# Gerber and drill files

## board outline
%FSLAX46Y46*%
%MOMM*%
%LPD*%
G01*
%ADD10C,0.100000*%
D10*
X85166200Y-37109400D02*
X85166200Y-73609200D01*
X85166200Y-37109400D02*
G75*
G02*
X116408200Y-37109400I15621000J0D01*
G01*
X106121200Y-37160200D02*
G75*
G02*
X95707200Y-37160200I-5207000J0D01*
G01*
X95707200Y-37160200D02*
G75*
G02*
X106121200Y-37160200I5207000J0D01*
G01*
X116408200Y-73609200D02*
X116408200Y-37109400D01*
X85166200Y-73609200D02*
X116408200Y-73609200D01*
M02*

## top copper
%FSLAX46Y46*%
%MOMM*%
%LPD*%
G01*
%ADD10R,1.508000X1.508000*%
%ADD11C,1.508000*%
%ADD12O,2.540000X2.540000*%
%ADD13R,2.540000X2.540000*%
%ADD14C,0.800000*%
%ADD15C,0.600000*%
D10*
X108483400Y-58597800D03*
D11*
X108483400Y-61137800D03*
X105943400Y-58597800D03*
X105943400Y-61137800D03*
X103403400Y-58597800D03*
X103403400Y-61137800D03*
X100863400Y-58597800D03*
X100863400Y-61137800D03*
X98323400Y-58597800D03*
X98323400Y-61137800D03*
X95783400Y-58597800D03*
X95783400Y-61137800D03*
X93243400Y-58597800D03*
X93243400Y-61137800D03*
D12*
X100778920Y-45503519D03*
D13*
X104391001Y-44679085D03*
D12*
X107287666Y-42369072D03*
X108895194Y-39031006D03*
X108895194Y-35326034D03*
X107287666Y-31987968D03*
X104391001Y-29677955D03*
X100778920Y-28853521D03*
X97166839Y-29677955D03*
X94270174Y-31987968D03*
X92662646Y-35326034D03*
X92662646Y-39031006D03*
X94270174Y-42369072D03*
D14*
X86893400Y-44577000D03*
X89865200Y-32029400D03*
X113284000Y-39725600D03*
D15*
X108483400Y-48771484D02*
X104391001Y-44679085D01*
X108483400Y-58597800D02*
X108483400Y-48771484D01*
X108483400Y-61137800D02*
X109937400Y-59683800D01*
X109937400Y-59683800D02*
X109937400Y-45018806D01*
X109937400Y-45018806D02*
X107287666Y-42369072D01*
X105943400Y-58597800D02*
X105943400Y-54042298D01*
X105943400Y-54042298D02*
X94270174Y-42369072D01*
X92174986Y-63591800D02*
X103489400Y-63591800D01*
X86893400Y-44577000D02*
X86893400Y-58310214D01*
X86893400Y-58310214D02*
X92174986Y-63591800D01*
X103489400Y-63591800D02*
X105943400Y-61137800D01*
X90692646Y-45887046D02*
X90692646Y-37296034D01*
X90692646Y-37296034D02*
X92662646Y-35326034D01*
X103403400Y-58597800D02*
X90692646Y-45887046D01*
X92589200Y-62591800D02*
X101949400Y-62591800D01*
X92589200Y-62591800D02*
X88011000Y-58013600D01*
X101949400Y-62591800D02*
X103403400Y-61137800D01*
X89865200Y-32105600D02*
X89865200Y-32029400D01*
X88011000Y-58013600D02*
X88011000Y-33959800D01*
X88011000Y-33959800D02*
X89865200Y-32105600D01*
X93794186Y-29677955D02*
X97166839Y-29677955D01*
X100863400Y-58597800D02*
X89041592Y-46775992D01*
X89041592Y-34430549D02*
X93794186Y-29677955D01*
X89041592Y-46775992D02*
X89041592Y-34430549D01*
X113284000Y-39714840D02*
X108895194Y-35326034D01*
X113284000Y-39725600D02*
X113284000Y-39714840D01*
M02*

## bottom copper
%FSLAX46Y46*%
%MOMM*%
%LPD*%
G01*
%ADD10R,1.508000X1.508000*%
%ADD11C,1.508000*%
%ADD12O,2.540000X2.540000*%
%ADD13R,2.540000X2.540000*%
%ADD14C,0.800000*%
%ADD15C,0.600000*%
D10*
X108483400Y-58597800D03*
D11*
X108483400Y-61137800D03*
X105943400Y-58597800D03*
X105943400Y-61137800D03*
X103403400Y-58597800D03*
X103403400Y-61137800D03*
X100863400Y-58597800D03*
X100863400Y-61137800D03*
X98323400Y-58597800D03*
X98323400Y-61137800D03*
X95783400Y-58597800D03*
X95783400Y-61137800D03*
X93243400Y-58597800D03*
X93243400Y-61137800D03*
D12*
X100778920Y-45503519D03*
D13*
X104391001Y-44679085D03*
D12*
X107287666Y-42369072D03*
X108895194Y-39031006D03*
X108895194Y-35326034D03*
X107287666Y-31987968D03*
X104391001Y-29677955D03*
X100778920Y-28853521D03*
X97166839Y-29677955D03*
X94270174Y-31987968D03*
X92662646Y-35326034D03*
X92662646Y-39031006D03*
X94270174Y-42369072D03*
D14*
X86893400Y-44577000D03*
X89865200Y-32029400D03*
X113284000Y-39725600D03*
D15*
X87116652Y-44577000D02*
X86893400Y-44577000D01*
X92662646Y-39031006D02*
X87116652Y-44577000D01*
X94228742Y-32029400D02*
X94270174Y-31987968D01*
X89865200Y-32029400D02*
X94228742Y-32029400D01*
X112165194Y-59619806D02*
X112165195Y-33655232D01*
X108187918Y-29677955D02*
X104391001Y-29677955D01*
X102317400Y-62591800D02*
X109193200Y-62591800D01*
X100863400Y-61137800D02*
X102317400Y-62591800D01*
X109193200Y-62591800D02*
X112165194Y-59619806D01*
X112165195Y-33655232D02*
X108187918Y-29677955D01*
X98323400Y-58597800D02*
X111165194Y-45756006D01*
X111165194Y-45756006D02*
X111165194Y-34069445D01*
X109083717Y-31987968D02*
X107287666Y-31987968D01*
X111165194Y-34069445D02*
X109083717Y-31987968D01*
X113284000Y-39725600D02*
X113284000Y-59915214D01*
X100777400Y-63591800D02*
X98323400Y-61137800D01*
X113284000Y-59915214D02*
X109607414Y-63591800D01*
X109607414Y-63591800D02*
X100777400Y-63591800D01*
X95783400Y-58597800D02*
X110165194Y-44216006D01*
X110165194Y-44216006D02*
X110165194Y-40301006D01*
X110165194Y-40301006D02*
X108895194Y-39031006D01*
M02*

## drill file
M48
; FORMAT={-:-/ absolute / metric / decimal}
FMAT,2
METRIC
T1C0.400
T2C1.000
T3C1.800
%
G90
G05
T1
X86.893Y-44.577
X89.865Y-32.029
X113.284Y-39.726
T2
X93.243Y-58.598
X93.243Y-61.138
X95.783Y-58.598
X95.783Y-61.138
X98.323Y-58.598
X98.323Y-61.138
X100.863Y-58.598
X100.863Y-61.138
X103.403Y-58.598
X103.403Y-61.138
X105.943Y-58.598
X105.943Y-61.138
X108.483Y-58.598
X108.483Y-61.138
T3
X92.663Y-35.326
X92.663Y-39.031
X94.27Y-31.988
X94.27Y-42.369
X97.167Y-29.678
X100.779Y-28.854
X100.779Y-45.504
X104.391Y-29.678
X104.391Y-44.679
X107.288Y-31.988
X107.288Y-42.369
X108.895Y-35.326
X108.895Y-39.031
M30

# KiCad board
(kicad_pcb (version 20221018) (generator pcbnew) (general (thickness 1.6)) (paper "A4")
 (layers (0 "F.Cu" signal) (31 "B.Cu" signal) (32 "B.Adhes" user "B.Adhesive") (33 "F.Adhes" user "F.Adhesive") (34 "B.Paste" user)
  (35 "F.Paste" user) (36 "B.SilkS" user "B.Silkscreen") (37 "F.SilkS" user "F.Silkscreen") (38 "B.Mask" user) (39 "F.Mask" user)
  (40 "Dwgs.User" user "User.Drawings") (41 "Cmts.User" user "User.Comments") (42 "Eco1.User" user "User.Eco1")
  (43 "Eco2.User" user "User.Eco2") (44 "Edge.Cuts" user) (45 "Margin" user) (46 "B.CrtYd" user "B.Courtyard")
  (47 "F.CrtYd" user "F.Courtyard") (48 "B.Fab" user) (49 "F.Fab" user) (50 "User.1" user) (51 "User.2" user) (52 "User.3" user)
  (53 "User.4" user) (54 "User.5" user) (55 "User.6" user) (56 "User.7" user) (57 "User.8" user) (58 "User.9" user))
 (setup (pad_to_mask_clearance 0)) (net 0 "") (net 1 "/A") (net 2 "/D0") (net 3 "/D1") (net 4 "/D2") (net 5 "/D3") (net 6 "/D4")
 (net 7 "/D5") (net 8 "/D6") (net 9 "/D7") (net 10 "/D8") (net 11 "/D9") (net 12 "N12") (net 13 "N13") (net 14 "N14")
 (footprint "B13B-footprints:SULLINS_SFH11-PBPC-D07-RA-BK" (layer "F.Cu") (at 100.8634 59.8678 180)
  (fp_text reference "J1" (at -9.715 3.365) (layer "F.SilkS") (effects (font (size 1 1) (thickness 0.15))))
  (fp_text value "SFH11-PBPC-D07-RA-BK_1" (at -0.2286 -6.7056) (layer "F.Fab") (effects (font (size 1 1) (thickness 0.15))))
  (pad "1" thru_hole rect (at -7.62 1.27 180) (size 1.508 1.508) (drill 1) (layers "*.Cu" "*.Mask") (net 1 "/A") (solder_mask_margin 0.102))
  (pad "2" thru_hole circle (at -7.62 -1.27 180) (size 1.508 1.508) (drill 1) (layers "*.Cu" "*.Mask") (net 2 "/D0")
   (solder_mask_margin 0.102))
  (pad "3" thru_hole circle (at -5.08 1.27 180) (size 1.508 1.508) (drill 1) (layers "*.Cu" "*.Mask") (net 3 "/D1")
   (solder_mask_margin 0.102))
  (pad "4" thru_hole circle (at -5.08 -1.27 180) (size 1.508 1.508) (drill 1) (layers "*.Cu" "*.Mask") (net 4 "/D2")
   (solder_mask_margin 0.102))
  (pad "5" thru_hole circle (at -2.54 1.27 180) (size 1.508 1.508) (drill 1) (layers "*.Cu" "*.Mask") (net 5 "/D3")
   (solder_mask_margin 0.102))
  (pad "6" thru_hole circle (at -2.54 -1.27 180) (size 1.508 1.508) (drill 1) (layers "*.Cu" "*.Mask") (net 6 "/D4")
   (solder_mask_margin 0.102))
  (pad "7" thru_hole circle (at 0 1.27 180) (size 1.508 1.508) (drill 1) (layers "*.Cu" "*.Mask") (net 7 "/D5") (solder_mask_margin 0.102))
  (pad "8" thru_hole circle (at 0 -1.27 180) (size 1.508 1.508) (drill 1) (layers "*.Cu" "*.Mask") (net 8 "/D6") (solder_mask_margin 0.102))
  (pad "9" thru_hole circle (at 2.54 1.27 180) (size 1.508 1.508) (drill 1) (layers "*.Cu" "*.Mask") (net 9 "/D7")
   (solder_mask_margin 0.102))
  (pad "10" thru_hole circle (at 2.54 -1.27 180) (size 1.508 1.508) (drill 1) (layers "*.Cu" "*.Mask") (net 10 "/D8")
   (solder_mask_margin 0.102))
  (pad "11" thru_hole circle (at 5.08 1.27 180) (size 1.508 1.508) (drill 1) (layers "*.Cu" "*.Mask") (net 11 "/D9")
   (solder_mask_margin 0.102))
  (pad "12" thru_hole circle (at 5.08 -1.27 180) (size 1.508 1.508) (drill 1) (layers "*.Cu" "*.Mask") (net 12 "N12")
   (solder_mask_margin 0.102))
  (pad "13" thru_hole circle (at 7.62 1.27 180) (size 1.508 1.508) (drill 1) (layers "*.Cu" "*.Mask") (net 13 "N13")
   (solder_mask_margin 0.102))
  (pad "14" thru_hole circle (at 7.62 -1.27 180) (size 1.508 1.508) (drill 1) (layers "*.Cu" "*.Mask") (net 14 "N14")
   (solder_mask_margin 0.102)))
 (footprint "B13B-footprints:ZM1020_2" (layer "F.Cu") (at 100.77892 37.17852)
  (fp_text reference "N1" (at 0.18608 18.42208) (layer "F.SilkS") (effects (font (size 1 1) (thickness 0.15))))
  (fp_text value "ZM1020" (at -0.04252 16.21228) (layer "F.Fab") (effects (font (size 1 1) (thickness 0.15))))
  (pad "1" thru_hole oval (at 0 8.324999) (size 2.54 2.54) (drill 1.8) (layers "*.Cu" "*.Mask") (thermal_bridge_angle 45))
  (pad "2" thru_hole rect (at 3.612081 7.500565) (size 2.54 2.54) (drill 1.8) (layers "*.Cu" "*.Mask") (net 1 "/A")
   (thermal_bridge_angle 45))
  (pad "3" thru_hole oval (at 6.508746 5.190552) (size 2.54 2.54) (drill 1.8) (layers "*.Cu" "*.Mask") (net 2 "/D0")
   (thermal_bridge_angle 45))
  (pad "4" thru_hole oval (at 8.116274 1.852486) (size 2.54 2.54) (drill 1.8) (layers "*.Cu" "*.Mask") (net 11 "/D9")
   (thermal_bridge_angle 45))
  (pad "5" thru_hole oval (at 8.116274 -1.852486) (size 2.54 2.54) (drill 1.8) (layers "*.Cu" "*.Mask") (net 10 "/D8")
   (thermal_bridge_angle 45))
  (pad "6" thru_hole oval (at 6.508746 -5.190552) (size 2.54 2.54) (drill 1.8) (layers "*.Cu" "*.Mask") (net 9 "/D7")
   (thermal_bridge_angle 45))
  (pad "7" thru_hole oval (at 3.612081 -7.500565) (size 2.54 2.54) (drill 1.8) (layers "*.Cu" "*.Mask") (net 8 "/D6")
   (thermal_bridge_angle 45))
  (pad "8" thru_hole oval (at 0 -8.324999) (size 2.54 2.54) (drill 1.8) (layers "*.Cu" "*.Mask") (thermal_bridge_angle 45))
  (pad "9" thru_hole oval (at -3.612081 -7.500565) (size 2.54 2.54) (drill 1.8) (layers "*.Cu" "*.Mask") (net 7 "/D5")
   (thermal_bridge_angle 45))
  (pad "10" thru_hole oval (at -6.508746 -5.190552) (size 2.54 2.54) (drill 1.8) (layers "*.Cu" "*.Mask") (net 6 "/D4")
   (thermal_bridge_angle 45))
  (pad "11" thru_hole oval (at -8.116274 -1.852486) (size 2.54 2.54) (drill 1.8) (layers "*.Cu" "*.Mask") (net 5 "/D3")
   (thermal_bridge_angle 45))
  (pad "12" thru_hole oval (at -8.116274 1.852486) (size 2.54 2.54) (drill 1.8) (layers "*.Cu" "*.Mask") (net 4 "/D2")
   (thermal_bridge_angle 45))
  (pad "13" thru_hole oval (at -6.508746 5.190552) (size 2.54 2.54) (drill 1.8) (layers "*.Cu" "*.Mask") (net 3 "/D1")
   (thermal_bridge_angle 45)))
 (gr_line (start 85.1662 37.1094) (end 85.1662 73.6092) (stroke (width 0.1) (type default)) (layer "Edge.Cuts"))
 (gr_arc (start 85.1662 37.1094) (mid 100.7872 21.4884) (end 116.4082 37.1094) (stroke (width 0.1) (type default)) (layer "Edge.Cuts"))
 (gr_arc (start 106.1212 37.1602) (mid 95.7072 37.1602) (end 106.1212 37.1602) (stroke (width 0.1) (type default)) (layer "Edge.Cuts"))
 (gr_line (start 116.4082 73.6092) (end 116.4082 37.1094) (stroke (width 0.1) (type default)) (layer "Edge.Cuts"))
 (gr_line (start 85.1662 73.6092) (end 116.4082 73.6092) (stroke (width 0.1) (type default)) (layer "Edge.Cuts"))
 (segment (start 108.4834 48.771484) (end 104.391001 44.679085) (width 0.6) (layer "F.Cu") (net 1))
 (segment (start 108.4834 58.5978) (end 108.4834 48.771484) (width 0.6) (layer "F.Cu") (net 1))
 (segment (start 108.4834 61.1378) (end 109.9374 59.6838) (width 0.6) (layer "F.Cu") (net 2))
 (segment (start 109.9374 59.6838) (end 109.9374 45.018806) (width 0.6) (layer "F.Cu") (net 2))
 (segment (start 109.9374 45.018806) (end 107.287666 42.369072) (width 0.6) (layer "F.Cu") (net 2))
 (segment (start 105.9434 58.5978) (end 105.9434 54.042298) (width 0.6) (layer "F.Cu") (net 3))
 (segment (start 105.9434 54.042298) (end 94.270174 42.369072) (width 0.6) (layer "F.Cu") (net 3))
 (segment (start 92.174986 63.5918) (end 103.4894 63.5918) (width 0.6) (layer "F.Cu") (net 4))
 (segment (start 86.8934 44.577) (end 86.8934 58.310214) (width 0.6) (layer "F.Cu") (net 4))
 (segment (start 86.8934 58.310214) (end 92.174986 63.5918) (width 0.6) (layer "F.Cu") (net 4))
 (segment (start 103.4894 63.5918) (end 105.9434 61.1378) (width 0.6) (layer "F.Cu") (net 4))
 (via (at 86.8934 44.577) (size 0.8) (drill 0.4) (layers "F.Cu" "B.Cu") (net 4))
 (segment (start 87.116652 44.577) (end 86.8934 44.577) (width 0.6) (layer "B.Cu") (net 4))
 (segment (start 92.662646 39.031006) (end 87.116652 44.577) (width 0.6) (layer "B.Cu") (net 4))
 (segment (start 90.692646 45.887046) (end 90.692646 37.296034) (width 0.6) (layer "F.Cu") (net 5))
 (segment (start 90.692646 37.296034) (end 92.662646 35.326034) (width 0.6) (layer "F.Cu") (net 5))
 (segment (start 103.4034 58.5978) (end 90.692646 45.887046) (width 0.6) (layer "F.Cu") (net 5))
 (segment (start 92.5892 62.5918) (end 101.9494 62.5918) (width 0.6) (layer "F.Cu") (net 6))
 (segment (start 92.5892 62.5918) (end 88.011 58.0136) (width 0.6) (layer "F.Cu") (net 6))
 (segment (start 101.9494 62.5918) (end 103.4034 61.1378) (width 0.6) (layer "F.Cu") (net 6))
 (segment (start 89.8652 32.1056) (end 89.8652 32.0294) (width 0.6) (layer "F.Cu") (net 6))
 (segment (start 88.011 58.0136) (end 88.011 33.9598) (width 0.6) (layer "F.Cu") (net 6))
 (segment (start 88.011 33.9598) (end 89.8652 32.1056) (width 0.6) (layer "F.Cu") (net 6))
 (via (at 89.8652 32.0294) (size 0.8) (drill 0.4) (layers "F.Cu" "B.Cu") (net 6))
 (segment (start 94.228742 32.0294) (end 94.270174 31.987968) (width 0.6) (layer "B.Cu") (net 6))
 (segment (start 89.8652 32.0294) (end 94.228742 32.0294) (width 0.6) (layer "B.Cu") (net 6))
 (segment (start 93.794186 29.677955) (end 97.166839 29.677955) (width 0.6) (layer "F.Cu") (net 7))
 (segment (start 100.8634 58.5978) (end 89.041592 46.775992) (width 0.6) (layer "F.Cu") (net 7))
 (segment (start 89.041592 34.430549) (end 93.794186 29.677955) (width 0.6) (layer "F.Cu") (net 7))
 (segment (start 89.041592 46.775992) (end 89.041592 34.430549) (width 0.6) (layer "F.Cu") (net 7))
 (segment (start 112.165194 59.619806) (end 112.165195 33.655232) (width 0.6) (layer "B.Cu") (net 8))
 (segment (start 108.187918 29.677955) (end 104.391001 29.677955) (width 0.6) (layer "B.Cu") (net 8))
 (segment (start 102.3174 62.5918) (end 109.1932 62.5918) (width 0.6) (layer "B.Cu") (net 8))
 (segment (start 100.8634 61.1378) (end 102.3174 62.5918) (width 0.6) (layer "B.Cu") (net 8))
 (segment (start 109.1932 62.5918) (end 112.165194 59.619806) (width 0.6) (layer "B.Cu") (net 8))
 (segment (start 112.165195 33.655232) (end 108.187918 29.677955) (width 0.6) (layer "B.Cu") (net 8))
 (segment (start 98.3234 58.5978) (end 111.165194 45.756006) (width 0.6) (layer "B.Cu") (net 9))
 (segment (start 111.165194 45.756006) (end 111.165194 34.069445) (width 0.6) (layer "B.Cu") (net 9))
 (segment (start 109.083717 31.987968) (end 107.287666 31.987968) (width 0.6) (layer "B.Cu") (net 9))
 (segment (start 111.165194 34.069445) (end 109.083717 31.987968) (width 0.6) (layer "B.Cu") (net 9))
 (segment (start 113.284 39.71484) (end 108.895194 35.326034) (width 0.6) (layer "F.Cu") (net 10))
 (segment (start 113.284 39.7256) (end 113.284 39.71484) (width 0.6) (layer "F.Cu") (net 10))
 (via (at 113.284 39.7256) (size 0.8) (drill 0.4) (layers "F.Cu" "B.Cu") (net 10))
 (segment (start 113.284 39.7256) (end 113.284 59.915214) (width 0.6) (layer "B.Cu") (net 10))
 (segment (start 100.7774 63.5918) (end 98.3234 61.1378) (width 0.6) (layer "B.Cu") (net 10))
 (segment (start 113.284 59.915214) (end 109.607414 63.5918) (width 0.6) (layer "B.Cu") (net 10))
 (segment (start 109.607414 63.5918) (end 100.7774 63.5918) (width 0.6) (layer "B.Cu") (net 10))
 (segment (start 95.7834 58.5978) (end 110.165194 44.216006) (width 0.6) (layer "B.Cu") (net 11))
 (segment (start 110.165194 44.216006) (end 110.165194 40.301006) (width 0.6) (layer "B.Cu") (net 11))
 (segment (start 110.165194 40.301006) (end 108.895194 39.031006) (width 0.6) (layer "B.Cu") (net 11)))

